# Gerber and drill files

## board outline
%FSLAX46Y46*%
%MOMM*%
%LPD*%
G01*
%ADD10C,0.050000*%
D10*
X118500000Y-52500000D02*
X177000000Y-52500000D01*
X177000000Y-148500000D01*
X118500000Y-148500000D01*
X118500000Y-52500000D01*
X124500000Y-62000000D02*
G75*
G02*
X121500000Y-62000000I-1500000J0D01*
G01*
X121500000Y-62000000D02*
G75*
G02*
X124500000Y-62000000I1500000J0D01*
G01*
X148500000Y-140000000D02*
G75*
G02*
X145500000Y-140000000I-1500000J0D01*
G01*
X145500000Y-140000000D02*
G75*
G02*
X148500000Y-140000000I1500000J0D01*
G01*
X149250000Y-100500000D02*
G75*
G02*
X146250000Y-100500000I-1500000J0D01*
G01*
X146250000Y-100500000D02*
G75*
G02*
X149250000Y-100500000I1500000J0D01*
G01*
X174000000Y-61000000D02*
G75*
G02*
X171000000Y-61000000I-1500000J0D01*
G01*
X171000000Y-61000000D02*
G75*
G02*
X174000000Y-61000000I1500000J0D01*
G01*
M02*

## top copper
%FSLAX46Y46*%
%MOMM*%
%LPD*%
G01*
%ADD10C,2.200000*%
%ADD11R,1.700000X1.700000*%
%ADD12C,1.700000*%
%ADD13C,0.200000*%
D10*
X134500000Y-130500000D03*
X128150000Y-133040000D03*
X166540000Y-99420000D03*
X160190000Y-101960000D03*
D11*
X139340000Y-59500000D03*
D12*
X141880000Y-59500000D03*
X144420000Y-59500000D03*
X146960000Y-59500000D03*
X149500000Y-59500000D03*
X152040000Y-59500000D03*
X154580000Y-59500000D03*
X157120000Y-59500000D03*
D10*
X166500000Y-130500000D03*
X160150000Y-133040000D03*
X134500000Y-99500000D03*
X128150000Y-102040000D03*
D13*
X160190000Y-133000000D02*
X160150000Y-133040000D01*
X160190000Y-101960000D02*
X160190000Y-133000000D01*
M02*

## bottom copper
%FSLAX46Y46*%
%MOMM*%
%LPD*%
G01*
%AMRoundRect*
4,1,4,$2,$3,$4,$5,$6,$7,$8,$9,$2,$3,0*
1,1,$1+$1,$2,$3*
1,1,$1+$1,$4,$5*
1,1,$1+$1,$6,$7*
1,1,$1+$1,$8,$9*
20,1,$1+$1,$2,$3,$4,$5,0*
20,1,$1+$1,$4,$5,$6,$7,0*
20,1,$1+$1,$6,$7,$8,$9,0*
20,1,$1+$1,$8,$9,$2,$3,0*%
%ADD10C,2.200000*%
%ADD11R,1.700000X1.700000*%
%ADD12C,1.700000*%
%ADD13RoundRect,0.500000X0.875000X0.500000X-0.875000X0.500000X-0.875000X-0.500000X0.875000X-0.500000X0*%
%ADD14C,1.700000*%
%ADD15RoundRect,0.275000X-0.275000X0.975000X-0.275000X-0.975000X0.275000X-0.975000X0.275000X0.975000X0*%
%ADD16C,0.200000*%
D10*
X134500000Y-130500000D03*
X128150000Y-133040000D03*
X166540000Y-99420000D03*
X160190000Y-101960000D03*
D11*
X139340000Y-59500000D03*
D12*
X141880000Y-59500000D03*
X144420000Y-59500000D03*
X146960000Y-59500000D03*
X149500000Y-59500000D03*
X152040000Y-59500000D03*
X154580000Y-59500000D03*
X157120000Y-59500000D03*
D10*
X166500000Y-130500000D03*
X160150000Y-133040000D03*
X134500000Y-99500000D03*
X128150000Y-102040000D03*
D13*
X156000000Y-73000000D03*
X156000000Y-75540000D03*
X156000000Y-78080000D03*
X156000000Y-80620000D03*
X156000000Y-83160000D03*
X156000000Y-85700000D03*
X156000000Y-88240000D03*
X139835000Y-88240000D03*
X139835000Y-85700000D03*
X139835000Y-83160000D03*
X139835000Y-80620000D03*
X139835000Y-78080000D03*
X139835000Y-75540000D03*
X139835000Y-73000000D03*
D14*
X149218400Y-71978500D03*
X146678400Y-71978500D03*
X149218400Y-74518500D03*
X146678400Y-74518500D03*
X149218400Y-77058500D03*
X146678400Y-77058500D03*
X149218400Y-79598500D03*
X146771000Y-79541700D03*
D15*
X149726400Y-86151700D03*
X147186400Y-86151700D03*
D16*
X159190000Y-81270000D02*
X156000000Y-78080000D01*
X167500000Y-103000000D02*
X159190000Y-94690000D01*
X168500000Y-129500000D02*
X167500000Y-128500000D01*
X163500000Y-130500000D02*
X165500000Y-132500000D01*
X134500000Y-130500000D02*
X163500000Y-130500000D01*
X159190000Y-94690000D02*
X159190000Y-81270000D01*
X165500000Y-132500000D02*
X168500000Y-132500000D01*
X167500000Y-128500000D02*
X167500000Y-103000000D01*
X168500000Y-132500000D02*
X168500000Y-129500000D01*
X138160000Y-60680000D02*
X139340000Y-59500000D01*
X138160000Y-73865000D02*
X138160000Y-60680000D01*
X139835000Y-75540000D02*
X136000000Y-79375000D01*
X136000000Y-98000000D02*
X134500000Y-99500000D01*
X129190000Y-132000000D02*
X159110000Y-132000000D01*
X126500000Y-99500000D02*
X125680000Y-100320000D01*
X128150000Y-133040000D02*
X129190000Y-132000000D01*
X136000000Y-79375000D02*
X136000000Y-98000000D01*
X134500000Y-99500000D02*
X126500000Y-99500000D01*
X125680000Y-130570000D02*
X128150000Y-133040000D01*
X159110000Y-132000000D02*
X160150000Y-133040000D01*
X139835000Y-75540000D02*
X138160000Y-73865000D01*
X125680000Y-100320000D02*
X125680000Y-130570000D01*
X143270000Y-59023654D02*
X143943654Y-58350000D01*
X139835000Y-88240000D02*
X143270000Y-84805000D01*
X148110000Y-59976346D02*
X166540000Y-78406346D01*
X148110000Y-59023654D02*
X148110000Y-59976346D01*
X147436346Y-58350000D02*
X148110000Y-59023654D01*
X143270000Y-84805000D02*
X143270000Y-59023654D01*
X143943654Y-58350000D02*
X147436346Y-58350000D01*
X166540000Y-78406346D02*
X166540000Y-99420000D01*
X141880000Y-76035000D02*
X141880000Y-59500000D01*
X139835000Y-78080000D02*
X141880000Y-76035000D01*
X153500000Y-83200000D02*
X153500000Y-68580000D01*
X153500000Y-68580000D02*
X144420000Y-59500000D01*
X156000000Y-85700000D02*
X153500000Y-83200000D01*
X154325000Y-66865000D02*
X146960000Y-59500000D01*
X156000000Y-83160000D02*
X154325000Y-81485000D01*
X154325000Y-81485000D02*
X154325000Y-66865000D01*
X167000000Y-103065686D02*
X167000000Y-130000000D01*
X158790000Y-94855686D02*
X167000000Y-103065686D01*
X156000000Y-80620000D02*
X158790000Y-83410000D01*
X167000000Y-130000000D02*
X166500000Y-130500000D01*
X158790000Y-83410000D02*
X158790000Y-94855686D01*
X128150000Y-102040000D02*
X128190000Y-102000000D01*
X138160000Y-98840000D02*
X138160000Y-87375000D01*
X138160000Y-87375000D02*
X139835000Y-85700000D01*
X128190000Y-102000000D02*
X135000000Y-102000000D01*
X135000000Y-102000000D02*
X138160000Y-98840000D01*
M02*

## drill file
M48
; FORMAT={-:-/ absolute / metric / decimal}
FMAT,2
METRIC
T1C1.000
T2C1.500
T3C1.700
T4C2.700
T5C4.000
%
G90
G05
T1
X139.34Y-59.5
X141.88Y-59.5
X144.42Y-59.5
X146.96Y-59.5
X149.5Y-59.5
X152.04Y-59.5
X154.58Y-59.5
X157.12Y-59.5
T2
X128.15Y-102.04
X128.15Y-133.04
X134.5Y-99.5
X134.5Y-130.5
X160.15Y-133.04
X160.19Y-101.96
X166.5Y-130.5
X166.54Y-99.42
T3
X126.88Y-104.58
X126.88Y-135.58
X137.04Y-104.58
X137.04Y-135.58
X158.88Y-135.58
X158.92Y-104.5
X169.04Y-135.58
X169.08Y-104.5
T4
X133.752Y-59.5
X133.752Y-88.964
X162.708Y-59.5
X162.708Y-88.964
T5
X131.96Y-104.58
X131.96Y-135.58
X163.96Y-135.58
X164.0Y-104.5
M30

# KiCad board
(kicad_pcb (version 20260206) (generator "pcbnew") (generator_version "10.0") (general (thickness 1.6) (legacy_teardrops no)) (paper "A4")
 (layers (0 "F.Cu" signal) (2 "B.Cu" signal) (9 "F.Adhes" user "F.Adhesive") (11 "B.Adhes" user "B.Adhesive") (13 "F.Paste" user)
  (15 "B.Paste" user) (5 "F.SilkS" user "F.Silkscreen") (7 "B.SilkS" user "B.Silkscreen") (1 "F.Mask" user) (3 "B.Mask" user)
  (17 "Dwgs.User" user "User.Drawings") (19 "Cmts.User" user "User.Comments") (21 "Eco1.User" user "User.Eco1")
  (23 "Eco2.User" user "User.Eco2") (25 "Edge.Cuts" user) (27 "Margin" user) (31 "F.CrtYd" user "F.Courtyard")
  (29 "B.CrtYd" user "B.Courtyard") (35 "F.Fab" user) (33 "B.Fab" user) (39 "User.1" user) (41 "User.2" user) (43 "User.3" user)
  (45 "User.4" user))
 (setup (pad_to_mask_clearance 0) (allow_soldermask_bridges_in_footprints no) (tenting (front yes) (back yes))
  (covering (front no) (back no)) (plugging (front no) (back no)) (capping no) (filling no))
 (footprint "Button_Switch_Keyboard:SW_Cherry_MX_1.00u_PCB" (layer "F.Cu") (at 134.5 130.5)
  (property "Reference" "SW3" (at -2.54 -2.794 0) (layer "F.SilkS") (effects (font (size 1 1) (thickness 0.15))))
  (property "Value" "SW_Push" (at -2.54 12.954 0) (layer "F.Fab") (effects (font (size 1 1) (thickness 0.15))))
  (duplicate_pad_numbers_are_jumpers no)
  (pad "" np_thru_hole circle (at -7.62 5.08) (size 1.7 1.7) (drill 1.7) (layers "*.Cu" "*.Mask"))
  (pad "" np_thru_hole circle (at -2.54 5.08) (size 4 4) (drill 4) (layers "*.Cu" "*.Mask"))
  (pad "" np_thru_hole circle (at 2.54 5.08) (size 1.7 1.7) (drill 1.7) (layers "*.Cu" "*.Mask"))
  (pad "1" thru_hole circle (at 0 0) (size 2.2 2.2) (drill 1.5) (layers "*.Cu" "*.Mask") (remove_unused_layers no)
   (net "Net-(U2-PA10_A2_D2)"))
  (pad "2" thru_hole circle (at -6.35 2.54) (size 2.2 2.2) (drill 1.5) (layers "*.Cu" "*.Mask") (remove_unused_layers no) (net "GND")))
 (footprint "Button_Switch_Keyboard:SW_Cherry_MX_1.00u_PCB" (layer "F.Cu") (at 166.54 99.42)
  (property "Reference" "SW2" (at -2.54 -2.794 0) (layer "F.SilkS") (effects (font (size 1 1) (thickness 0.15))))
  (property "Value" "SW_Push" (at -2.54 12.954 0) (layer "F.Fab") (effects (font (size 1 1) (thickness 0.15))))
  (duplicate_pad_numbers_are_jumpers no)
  (pad "" np_thru_hole circle (at -7.62 5.08) (size 1.7 1.7) (drill 1.7) (layers "*.Cu" "*.Mask"))
  (pad "" np_thru_hole circle (at -2.54 5.08) (size 4 4) (drill 4) (layers "*.Cu" "*.Mask"))
  (pad "" np_thru_hole circle (at 2.54 5.08) (size 1.7 1.7) (drill 1.7) (layers "*.Cu" "*.Mask"))
  (pad "1" thru_hole circle (at 0 0) (size 2.2 2.2) (drill 1.5) (layers "*.Cu" "*.Mask") (remove_unused_layers no)
   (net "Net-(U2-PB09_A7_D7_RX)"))
  (pad "2" thru_hole circle (at -6.35 2.54) (size 2.2 2.2) (drill 1.5) (layers "*.Cu" "*.Mask") (remove_unused_layers no) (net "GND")))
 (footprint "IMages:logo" (layer "F.Cu") (at 148 105.5)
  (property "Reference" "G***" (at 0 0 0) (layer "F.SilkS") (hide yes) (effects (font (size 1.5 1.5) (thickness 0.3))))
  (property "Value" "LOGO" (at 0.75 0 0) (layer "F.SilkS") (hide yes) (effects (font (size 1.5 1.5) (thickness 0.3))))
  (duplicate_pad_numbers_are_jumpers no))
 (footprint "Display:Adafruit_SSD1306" (layer "F.Cu") (at 139.34 59.5)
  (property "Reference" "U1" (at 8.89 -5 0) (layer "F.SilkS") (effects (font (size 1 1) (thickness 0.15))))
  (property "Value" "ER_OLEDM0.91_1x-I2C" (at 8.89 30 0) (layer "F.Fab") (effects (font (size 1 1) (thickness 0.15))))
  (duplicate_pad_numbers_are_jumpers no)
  (pad "" np_thru_hole circle (at -5.588 0) (size 2.7 2.7) (drill 2.7) (layers "*.Cu" "*.Mask"))
  (pad "" np_thru_hole circle (at -5.588 29.464) (size 2.7 2.7) (drill 2.7) (layers "*.Cu" "*.Mask"))
  (pad "" np_thru_hole circle (at 23.368 0) (size 2.7 2.7) (drill 2.7) (layers "*.Cu" "*.Mask"))
  (pad "" np_thru_hole circle (at 23.368 29.464) (size 2.7 2.7) (drill 2.7) (layers "*.Cu" "*.Mask"))
  (pad "1" thru_hole rect (at 0 0) (size 1.7 1.7) (drill 1) (layers "*.Cu" "*.Mask") (remove_unused_layers no) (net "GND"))
  (pad "2" thru_hole circle (at 2.54 0) (size 1.7 1.7) (drill 1) (layers "*.Cu" "*.Mask") (remove_unused_layers no) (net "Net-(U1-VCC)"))
  (pad "3" thru_hole circle (at 5.08 0) (size 1.7 1.7) (drill 1) (layers "*.Cu" "*.Mask") (remove_unused_layers no) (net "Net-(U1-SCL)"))
  (pad "4" thru_hole circle (at 7.62 0) (size 1.7 1.7) (drill 1) (layers "*.Cu" "*.Mask") (remove_unused_layers no) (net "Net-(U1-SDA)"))
  (pad "5" thru_hole circle (at 10.16 0) (size 1.7 1.7) (drill 1) (layers "*.Cu" "*.Mask") (remove_unused_layers no))
  (pad "6" thru_hole circle (at 12.7 0) (size 1.7 1.7) (drill 1) (layers "*.Cu" "*.Mask") (remove_unused_layers no))
  (pad "7" thru_hole circle (at 15.24 0) (size 1.7 1.7) (drill 1) (layers "*.Cu" "*.Mask") (remove_unused_layers no))
  (pad "8" thru_hole circle (at 17.78 0) (size 1.7 1.7) (drill 1) (layers "*.Cu" "*.Mask") (remove_unused_layers no)))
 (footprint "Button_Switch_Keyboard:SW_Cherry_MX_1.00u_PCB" (layer "F.Cu") (at 166.5 130.5)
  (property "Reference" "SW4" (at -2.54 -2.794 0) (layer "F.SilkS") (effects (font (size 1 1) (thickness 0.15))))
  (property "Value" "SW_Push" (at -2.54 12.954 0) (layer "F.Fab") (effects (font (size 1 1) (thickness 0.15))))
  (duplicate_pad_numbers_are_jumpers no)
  (pad "" np_thru_hole circle (at -7.62 5.08) (size 1.7 1.7) (drill 1.7) (layers "*.Cu" "*.Mask"))
  (pad "" np_thru_hole circle (at -2.54 5.08) (size 4 4) (drill 4) (layers "*.Cu" "*.Mask"))
  (pad "" np_thru_hole circle (at 2.54 5.08) (size 1.7 1.7) (drill 1.7) (layers "*.Cu" "*.Mask"))
  (pad "1" thru_hole circle (at 0 0) (size 2.2 2.2) (drill 1.5) (layers "*.Cu" "*.Mask") (remove_unused_layers no)
   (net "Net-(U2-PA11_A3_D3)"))
  (pad "2" thru_hole circle (at -6.35 2.54) (size 2.2 2.2) (drill 1.5) (layers "*.Cu" "*.Mask") (remove_unused_layers no) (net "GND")))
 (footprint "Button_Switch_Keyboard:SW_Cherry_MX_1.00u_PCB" (layer "F.Cu") (at 134.5 99.5)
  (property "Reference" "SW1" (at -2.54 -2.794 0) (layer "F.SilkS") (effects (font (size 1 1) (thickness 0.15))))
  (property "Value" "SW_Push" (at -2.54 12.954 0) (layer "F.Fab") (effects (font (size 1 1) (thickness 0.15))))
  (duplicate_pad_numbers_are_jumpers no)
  (pad "" np_thru_hole circle (at -7.62 5.08) (size 1.7 1.7) (drill 1.7) (layers "*.Cu" "*.Mask"))
  (pad "" np_thru_hole circle (at -2.54 5.08) (size 4 4) (drill 4) (layers "*.Cu" "*.Mask"))
  (pad "" np_thru_hole circle (at 2.54 5.08) (size 1.7 1.7) (drill 1.7) (layers "*.Cu" "*.Mask"))
  (pad "1" thru_hole circle (at 0 0) (size 2.2 2.2) (drill 1.5) (layers "*.Cu" "*.Mask") (remove_unused_layers no) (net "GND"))
  (pad "2" thru_hole circle (at -6.35 2.54) (size 2.2 2.2) (drill 1.5) (layers "*.Cu" "*.Mask") (remove_unused_layers no)
   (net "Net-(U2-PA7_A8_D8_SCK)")))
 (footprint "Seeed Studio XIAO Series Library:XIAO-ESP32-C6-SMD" (layer "B.Cu") (at 156.835 91.12 180)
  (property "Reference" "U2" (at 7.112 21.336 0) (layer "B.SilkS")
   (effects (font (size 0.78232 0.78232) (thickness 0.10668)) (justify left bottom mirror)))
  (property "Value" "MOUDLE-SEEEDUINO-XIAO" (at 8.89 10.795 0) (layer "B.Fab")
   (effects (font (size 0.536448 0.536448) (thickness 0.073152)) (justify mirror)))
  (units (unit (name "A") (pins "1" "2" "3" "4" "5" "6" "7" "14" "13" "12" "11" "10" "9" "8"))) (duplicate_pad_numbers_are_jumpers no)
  (pad "1" smd roundrect (at 0.835 18.12 180) (size 2.75 2) (layers "B.Cu" "B.Mask" "B.Paste") (roundrect_rratio 0.25)
   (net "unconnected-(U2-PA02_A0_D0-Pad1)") (solder_mask_margin 0.0508) (thermal_bridge_angle 45))
  (pad "2" smd roundrect (at 0.835 15.58 180) (size 2.75 2) (layers "B.Cu" "B.Mask" "B.Paste") (roundrect_rratio 0.25)
   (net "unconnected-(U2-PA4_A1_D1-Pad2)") (solder_mask_margin 0.0508) (thermal_bridge_angle 45))
  (pad "3" smd roundrect (at 0.835 13.04 180) (size 2.75 2) (layers "B.Cu" "B.Mask" "B.Paste") (roundrect_rratio 0.25)
   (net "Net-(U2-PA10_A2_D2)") (solder_mask_margin 0.0508) (thermal_bridge_angle 45))
  (pad "4" smd roundrect (at 0.835 10.5 180) (size 2.75 2) (layers "B.Cu" "B.Mask" "B.Paste") (roundrect_rratio 0.25)
   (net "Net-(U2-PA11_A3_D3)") (solder_mask_margin 0.0508) (thermal_bridge_angle 45))
  (pad "5" smd roundrect (at 0.835 7.96 180) (size 2.75 2) (layers "B.Cu" "B.Mask" "B.Paste") (roundrect_rratio 0.25) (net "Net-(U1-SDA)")
   (solder_mask_margin 0.0508) (thermal_bridge_angle 45))
  (pad "6" smd roundrect (at 0.835 5.42 180) (size 2.75 2) (layers "B.Cu" "B.Mask" "B.Paste") (roundrect_rratio 0.25) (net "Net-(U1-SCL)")
   (solder_mask_margin 0.0508) (thermal_bridge_angle 45))
  (pad "7" smd roundrect (at 0.835 2.88 180) (size 2.75 2) (layers "B.Cu" "B.Mask" "B.Paste") (roundrect_rratio 0.25)
   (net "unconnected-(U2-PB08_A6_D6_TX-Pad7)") (solder_mask_margin 0.0508) (thermal_bridge_angle 45))
  (pad "8" smd roundrect (at 17 2.88 180) (size 2.75 2) (layers "B.Cu" "B.Mask" "B.Paste") (roundrect_rratio 0.25)
   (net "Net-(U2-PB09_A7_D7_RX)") (solder_mask_margin 0.0508) (thermal_bridge_angle 45))
  (pad "9" smd roundrect (at 17 5.42 180) (size 2.75 2) (layers "B.Cu" "B.Mask" "B.Paste") (roundrect_rratio 0.25)
   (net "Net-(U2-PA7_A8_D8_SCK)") (solder_mask_margin 0.0508) (thermal_bridge_angle 45))
  (pad "10" smd roundrect (at 17 7.96 180) (size 2.75 2) (layers "B.Cu" "B.Mask" "B.Paste") (roundrect_rratio 0.25)
   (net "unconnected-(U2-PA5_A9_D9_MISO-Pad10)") (solder_mask_margin 0.0508) (thermal_bridge_angle 45))
  (pad "11" smd roundrect (at 17 10.5 180) (size 2.75 2) (layers "B.Cu" "B.Mask" "B.Paste") (roundrect_rratio 0.25)
   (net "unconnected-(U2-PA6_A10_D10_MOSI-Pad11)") (solder_mask_margin 0.0508) (thermal_bridge_angle 45))
  (pad "12" smd roundrect (at 17 13.04 180) (size 2.75 2) (layers "B.Cu" "B.Mask" "B.Paste") (roundrect_rratio 0.25) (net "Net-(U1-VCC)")
   (solder_mask_margin 0.0508) (thermal_bridge_angle 45))
  (pad "13" smd roundrect (at 17 15.58 180) (size 2.75 2) (layers "B.Cu" "B.Mask" "B.Paste") (roundrect_rratio 0.25) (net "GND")
   (solder_mask_margin 0.0508) (thermal_bridge_angle 45))
  (pad "14" smd roundrect (at 17 18.12 180) (size 2.75 2) (layers "B.Cu" "B.Mask" "B.Paste") (roundrect_rratio 0.25)
   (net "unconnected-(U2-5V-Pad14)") (solder_mask_margin 0.0508) (thermal_bridge_angle 45))
  (pad "15" smd circle (at 7.6166 19.1415 180) (size 1.7 1.7) (layers "B.Cu" "B.Mask" "B.Paste"))
  (pad "16" smd circle (at 10.1566 19.1415 180) (size 1.7 1.7) (layers "B.Cu" "B.Mask" "B.Paste"))
  (pad "17" smd circle (at 7.6166 16.6015 180) (size 1.7 1.7) (layers "B.Cu" "B.Mask" "B.Paste"))
  (pad "18" smd circle (at 10.1566 16.6015 180) (size 1.7 1.7) (layers "B.Cu" "B.Mask" "B.Paste"))
  (pad "19" smd circle (at 7.6166 14.0615 180) (size 1.7 1.7) (layers "B.Cu" "B.Mask" "B.Paste"))
  (pad "20" smd circle (at 10.1566 14.0615 180) (size 1.7 1.7) (layers "B.Cu" "B.Mask" "B.Paste"))
  (pad "21" smd circle (at 7.6166 11.5215 180) (size 1.7 1.7) (layers "B.Cu" "B.Mask" "B.Paste"))
  (pad "22" smd circle (at 10.064 11.5783 180) (size 1.7 1.7) (layers "B.Cu" "B.Mask" "B.Paste"))
  (pad "23" smd roundrect (at 7.1086 4.9683 270) (size 2.5 1.1) (layers "B.Cu" "B.Mask" "B.Paste") (roundrect_rratio 0.25)
   (thermal_bridge_angle 45))
  (pad "24" smd roundrect (at 9.6486 4.9683 270) (size 2.5 1.1) (layers "B.Cu" "B.Mask" "B.Paste") (roundrect_rratio 0.25)
   (thermal_bridge_angle 45)))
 (gr_rect (start 118.5 52.5) (end 177 148.5) (stroke (width 0.05) (type default)) (fill no) (layer "Edge.Cuts"))
 (gr_circle (center 123 62) (end 123 60.5) (stroke (width 0.05) (type default)) (fill no) (layer "Edge.Cuts"))
 (gr_circle (center 147 140) (end 145.5 140) (stroke (width 0.05) (type default)) (fill no) (layer "Edge.Cuts"))
 (gr_circle (center 147.75 100.5) (end 147.75 99) (stroke (width 0.05) (type default)) (fill no) (layer "Edge.Cuts"))
 (gr_circle (center 172.5 61) (end 172.5 59.5) (stroke (width 0.05) (type default)) (fill no) (layer "Edge.Cuts"))
 (segment (start 159.19 81.27) (end 156 78.08) (width 0.2) (layer "B.Cu") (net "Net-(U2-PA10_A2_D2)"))
 (segment (start 167.5 103) (end 159.19 94.69) (width 0.2) (layer "B.Cu") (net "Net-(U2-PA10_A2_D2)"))
 (segment (start 168.5 129.5) (end 167.5 128.5) (width 0.2) (layer "B.Cu") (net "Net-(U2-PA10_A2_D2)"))
 (segment (start 163.5 130.5) (end 165.5 132.5) (width 0.2) (layer "B.Cu") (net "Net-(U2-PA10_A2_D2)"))
 (segment (start 134.5 130.5) (end 163.5 130.5) (width 0.2) (layer "B.Cu") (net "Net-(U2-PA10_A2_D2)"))
 (segment (start 159.19 94.69) (end 159.19 81.27) (width 0.2) (layer "B.Cu") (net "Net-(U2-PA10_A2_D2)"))
 (segment (start 165.5 132.5) (end 168.5 132.5) (width 0.2) (layer "B.Cu") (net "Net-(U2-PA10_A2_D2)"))
 (segment (start 167.5 128.5) (end 167.5 103) (width 0.2) (layer "B.Cu") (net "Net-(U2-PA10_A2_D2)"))
 (segment (start 168.5 132.5) (end 168.5 129.5) (width 0.2) (layer "B.Cu") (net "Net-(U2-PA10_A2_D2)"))
 (segment (start 160.19 133) (end 160.15 133.04) (width 0.2) (layer "F.Cu") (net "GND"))
 (segment (start 160.19 101.96) (end 160.19 133) (width 0.2) (layer "F.Cu") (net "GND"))
 (segment (start 138.16 60.68) (end 139.34 59.5) (width 0.2) (layer "B.Cu") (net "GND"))
 (segment (start 138.16 73.865) (end 138.16 60.68) (width 0.2) (layer "B.Cu") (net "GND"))
 (segment (start 139.835 75.54) (end 136 79.375) (width 0.2) (layer "B.Cu") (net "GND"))
 (segment (start 136 98) (end 134.5 99.5) (width 0.2) (layer "B.Cu") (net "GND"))
 (segment (start 129.19 132) (end 159.11 132) (width 0.2) (layer "B.Cu") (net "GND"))
 (segment (start 126.5 99.5) (end 125.68 100.32) (width 0.2) (layer "B.Cu") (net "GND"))
 (segment (start 128.15 133.04) (end 129.19 132) (width 0.2) (layer "B.Cu") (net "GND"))
 (segment (start 136 79.375) (end 136 98) (width 0.2) (layer "B.Cu") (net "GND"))
 (segment (start 134.5 99.5) (end 126.5 99.5) (width 0.2) (layer "B.Cu") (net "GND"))
 (segment (start 125.68 130.57) (end 128.15 133.04) (width 0.2) (layer "B.Cu") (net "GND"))
 (segment (start 159.11 132) (end 160.15 133.04) (width 0.2) (layer "B.Cu") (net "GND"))
 (segment (start 139.835 75.54) (end 138.16 73.865) (width 0.2) (layer "B.Cu") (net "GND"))
 (segment (start 125.68 100.32) (end 125.68 130.57) (width 0.2) (layer "B.Cu") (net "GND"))
 (segment (start 143.27 59.023654) (end 143.943654 58.35) (width 0.2) (layer "B.Cu") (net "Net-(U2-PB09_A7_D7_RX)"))
 (segment (start 139.835 88.24) (end 143.27 84.805) (width 0.2) (layer "B.Cu") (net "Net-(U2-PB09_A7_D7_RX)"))
 (segment (start 148.11 59.976346) (end 166.54 78.406346) (width 0.2) (layer "B.Cu") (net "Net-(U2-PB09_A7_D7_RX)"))
 (segment (start 148.11 59.023654) (end 148.11 59.976346) (width 0.2) (layer "B.Cu") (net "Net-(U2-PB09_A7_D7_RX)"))
 (segment (start 147.436346 58.35) (end 148.11 59.023654) (width 0.2) (layer "B.Cu") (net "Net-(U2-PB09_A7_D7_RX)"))
 (segment (start 143.27 84.805) (end 143.27 59.023654) (width 0.2) (layer "B.Cu") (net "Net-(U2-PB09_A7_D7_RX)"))
 (segment (start 143.943654 58.35) (end 147.436346 58.35) (width 0.2) (layer "B.Cu") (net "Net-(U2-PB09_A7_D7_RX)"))
 (segment (start 166.54 78.406346) (end 166.54 99.42) (width 0.2) (layer "B.Cu") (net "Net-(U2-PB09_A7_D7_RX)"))
 (segment (start 141.88 76.035) (end 141.88 59.5) (width 0.2) (layer "B.Cu") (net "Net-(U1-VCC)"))
 (segment (start 139.835 78.08) (end 141.88 76.035) (width 0.2) (layer "B.Cu") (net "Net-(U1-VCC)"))
 (segment (start 153.5 83.2) (end 153.5 68.58) (width 0.2) (layer "B.Cu") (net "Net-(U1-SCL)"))
 (segment (start 153.5 68.58) (end 144.42 59.5) (width 0.2) (layer "B.Cu") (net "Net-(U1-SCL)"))
 (segment (start 156 85.7) (end 153.5 83.2) (width 0.2) (layer "B.Cu") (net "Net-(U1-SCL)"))
 (segment (start 154.325 66.865) (end 146.96 59.5) (width 0.2) (layer "B.Cu") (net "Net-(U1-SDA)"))
 (segment (start 156 83.16) (end 154.325 81.485) (width 0.2) (layer "B.Cu") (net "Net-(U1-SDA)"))
 (segment (start 154.325 81.485) (end 154.325 66.865) (width 0.2) (layer "B.Cu") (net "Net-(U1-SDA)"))
 (segment (start 167 103.065686) (end 167 130) (width 0.2) (layer "B.Cu") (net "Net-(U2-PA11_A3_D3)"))
 (segment (start 158.79 94.855686) (end 167 103.065686) (width 0.2) (layer "B.Cu") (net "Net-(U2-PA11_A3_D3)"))
 (segment (start 156 80.62) (end 158.79 83.41) (width 0.2) (layer "B.Cu") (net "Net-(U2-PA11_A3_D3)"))
 (segment (start 167 130) (end 166.5 130.5) (width 0.2) (layer "B.Cu") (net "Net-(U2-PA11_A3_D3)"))
 (segment (start 158.79 83.41) (end 158.79 94.855686) (width 0.2) (layer "B.Cu") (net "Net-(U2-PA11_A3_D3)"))
 (segment (start 128.15 102.04) (end 128.19 102) (width 0.2) (layer "B.Cu") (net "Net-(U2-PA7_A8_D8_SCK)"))
 (segment (start 138.16 98.84) (end 138.16 87.375) (width 0.2) (layer "B.Cu") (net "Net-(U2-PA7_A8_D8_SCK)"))
 (segment (start 138.16 87.375) (end 139.835 85.7) (width 0.2) (layer "B.Cu") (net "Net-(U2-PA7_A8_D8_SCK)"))
 (segment (start 128.19 102) (end 135 102) (width 0.2) (layer "B.Cu") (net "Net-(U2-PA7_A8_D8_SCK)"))
 (segment (start 135 102) (end 138.16 98.84) (width 0.2) (layer "B.Cu") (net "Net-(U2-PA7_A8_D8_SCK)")))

